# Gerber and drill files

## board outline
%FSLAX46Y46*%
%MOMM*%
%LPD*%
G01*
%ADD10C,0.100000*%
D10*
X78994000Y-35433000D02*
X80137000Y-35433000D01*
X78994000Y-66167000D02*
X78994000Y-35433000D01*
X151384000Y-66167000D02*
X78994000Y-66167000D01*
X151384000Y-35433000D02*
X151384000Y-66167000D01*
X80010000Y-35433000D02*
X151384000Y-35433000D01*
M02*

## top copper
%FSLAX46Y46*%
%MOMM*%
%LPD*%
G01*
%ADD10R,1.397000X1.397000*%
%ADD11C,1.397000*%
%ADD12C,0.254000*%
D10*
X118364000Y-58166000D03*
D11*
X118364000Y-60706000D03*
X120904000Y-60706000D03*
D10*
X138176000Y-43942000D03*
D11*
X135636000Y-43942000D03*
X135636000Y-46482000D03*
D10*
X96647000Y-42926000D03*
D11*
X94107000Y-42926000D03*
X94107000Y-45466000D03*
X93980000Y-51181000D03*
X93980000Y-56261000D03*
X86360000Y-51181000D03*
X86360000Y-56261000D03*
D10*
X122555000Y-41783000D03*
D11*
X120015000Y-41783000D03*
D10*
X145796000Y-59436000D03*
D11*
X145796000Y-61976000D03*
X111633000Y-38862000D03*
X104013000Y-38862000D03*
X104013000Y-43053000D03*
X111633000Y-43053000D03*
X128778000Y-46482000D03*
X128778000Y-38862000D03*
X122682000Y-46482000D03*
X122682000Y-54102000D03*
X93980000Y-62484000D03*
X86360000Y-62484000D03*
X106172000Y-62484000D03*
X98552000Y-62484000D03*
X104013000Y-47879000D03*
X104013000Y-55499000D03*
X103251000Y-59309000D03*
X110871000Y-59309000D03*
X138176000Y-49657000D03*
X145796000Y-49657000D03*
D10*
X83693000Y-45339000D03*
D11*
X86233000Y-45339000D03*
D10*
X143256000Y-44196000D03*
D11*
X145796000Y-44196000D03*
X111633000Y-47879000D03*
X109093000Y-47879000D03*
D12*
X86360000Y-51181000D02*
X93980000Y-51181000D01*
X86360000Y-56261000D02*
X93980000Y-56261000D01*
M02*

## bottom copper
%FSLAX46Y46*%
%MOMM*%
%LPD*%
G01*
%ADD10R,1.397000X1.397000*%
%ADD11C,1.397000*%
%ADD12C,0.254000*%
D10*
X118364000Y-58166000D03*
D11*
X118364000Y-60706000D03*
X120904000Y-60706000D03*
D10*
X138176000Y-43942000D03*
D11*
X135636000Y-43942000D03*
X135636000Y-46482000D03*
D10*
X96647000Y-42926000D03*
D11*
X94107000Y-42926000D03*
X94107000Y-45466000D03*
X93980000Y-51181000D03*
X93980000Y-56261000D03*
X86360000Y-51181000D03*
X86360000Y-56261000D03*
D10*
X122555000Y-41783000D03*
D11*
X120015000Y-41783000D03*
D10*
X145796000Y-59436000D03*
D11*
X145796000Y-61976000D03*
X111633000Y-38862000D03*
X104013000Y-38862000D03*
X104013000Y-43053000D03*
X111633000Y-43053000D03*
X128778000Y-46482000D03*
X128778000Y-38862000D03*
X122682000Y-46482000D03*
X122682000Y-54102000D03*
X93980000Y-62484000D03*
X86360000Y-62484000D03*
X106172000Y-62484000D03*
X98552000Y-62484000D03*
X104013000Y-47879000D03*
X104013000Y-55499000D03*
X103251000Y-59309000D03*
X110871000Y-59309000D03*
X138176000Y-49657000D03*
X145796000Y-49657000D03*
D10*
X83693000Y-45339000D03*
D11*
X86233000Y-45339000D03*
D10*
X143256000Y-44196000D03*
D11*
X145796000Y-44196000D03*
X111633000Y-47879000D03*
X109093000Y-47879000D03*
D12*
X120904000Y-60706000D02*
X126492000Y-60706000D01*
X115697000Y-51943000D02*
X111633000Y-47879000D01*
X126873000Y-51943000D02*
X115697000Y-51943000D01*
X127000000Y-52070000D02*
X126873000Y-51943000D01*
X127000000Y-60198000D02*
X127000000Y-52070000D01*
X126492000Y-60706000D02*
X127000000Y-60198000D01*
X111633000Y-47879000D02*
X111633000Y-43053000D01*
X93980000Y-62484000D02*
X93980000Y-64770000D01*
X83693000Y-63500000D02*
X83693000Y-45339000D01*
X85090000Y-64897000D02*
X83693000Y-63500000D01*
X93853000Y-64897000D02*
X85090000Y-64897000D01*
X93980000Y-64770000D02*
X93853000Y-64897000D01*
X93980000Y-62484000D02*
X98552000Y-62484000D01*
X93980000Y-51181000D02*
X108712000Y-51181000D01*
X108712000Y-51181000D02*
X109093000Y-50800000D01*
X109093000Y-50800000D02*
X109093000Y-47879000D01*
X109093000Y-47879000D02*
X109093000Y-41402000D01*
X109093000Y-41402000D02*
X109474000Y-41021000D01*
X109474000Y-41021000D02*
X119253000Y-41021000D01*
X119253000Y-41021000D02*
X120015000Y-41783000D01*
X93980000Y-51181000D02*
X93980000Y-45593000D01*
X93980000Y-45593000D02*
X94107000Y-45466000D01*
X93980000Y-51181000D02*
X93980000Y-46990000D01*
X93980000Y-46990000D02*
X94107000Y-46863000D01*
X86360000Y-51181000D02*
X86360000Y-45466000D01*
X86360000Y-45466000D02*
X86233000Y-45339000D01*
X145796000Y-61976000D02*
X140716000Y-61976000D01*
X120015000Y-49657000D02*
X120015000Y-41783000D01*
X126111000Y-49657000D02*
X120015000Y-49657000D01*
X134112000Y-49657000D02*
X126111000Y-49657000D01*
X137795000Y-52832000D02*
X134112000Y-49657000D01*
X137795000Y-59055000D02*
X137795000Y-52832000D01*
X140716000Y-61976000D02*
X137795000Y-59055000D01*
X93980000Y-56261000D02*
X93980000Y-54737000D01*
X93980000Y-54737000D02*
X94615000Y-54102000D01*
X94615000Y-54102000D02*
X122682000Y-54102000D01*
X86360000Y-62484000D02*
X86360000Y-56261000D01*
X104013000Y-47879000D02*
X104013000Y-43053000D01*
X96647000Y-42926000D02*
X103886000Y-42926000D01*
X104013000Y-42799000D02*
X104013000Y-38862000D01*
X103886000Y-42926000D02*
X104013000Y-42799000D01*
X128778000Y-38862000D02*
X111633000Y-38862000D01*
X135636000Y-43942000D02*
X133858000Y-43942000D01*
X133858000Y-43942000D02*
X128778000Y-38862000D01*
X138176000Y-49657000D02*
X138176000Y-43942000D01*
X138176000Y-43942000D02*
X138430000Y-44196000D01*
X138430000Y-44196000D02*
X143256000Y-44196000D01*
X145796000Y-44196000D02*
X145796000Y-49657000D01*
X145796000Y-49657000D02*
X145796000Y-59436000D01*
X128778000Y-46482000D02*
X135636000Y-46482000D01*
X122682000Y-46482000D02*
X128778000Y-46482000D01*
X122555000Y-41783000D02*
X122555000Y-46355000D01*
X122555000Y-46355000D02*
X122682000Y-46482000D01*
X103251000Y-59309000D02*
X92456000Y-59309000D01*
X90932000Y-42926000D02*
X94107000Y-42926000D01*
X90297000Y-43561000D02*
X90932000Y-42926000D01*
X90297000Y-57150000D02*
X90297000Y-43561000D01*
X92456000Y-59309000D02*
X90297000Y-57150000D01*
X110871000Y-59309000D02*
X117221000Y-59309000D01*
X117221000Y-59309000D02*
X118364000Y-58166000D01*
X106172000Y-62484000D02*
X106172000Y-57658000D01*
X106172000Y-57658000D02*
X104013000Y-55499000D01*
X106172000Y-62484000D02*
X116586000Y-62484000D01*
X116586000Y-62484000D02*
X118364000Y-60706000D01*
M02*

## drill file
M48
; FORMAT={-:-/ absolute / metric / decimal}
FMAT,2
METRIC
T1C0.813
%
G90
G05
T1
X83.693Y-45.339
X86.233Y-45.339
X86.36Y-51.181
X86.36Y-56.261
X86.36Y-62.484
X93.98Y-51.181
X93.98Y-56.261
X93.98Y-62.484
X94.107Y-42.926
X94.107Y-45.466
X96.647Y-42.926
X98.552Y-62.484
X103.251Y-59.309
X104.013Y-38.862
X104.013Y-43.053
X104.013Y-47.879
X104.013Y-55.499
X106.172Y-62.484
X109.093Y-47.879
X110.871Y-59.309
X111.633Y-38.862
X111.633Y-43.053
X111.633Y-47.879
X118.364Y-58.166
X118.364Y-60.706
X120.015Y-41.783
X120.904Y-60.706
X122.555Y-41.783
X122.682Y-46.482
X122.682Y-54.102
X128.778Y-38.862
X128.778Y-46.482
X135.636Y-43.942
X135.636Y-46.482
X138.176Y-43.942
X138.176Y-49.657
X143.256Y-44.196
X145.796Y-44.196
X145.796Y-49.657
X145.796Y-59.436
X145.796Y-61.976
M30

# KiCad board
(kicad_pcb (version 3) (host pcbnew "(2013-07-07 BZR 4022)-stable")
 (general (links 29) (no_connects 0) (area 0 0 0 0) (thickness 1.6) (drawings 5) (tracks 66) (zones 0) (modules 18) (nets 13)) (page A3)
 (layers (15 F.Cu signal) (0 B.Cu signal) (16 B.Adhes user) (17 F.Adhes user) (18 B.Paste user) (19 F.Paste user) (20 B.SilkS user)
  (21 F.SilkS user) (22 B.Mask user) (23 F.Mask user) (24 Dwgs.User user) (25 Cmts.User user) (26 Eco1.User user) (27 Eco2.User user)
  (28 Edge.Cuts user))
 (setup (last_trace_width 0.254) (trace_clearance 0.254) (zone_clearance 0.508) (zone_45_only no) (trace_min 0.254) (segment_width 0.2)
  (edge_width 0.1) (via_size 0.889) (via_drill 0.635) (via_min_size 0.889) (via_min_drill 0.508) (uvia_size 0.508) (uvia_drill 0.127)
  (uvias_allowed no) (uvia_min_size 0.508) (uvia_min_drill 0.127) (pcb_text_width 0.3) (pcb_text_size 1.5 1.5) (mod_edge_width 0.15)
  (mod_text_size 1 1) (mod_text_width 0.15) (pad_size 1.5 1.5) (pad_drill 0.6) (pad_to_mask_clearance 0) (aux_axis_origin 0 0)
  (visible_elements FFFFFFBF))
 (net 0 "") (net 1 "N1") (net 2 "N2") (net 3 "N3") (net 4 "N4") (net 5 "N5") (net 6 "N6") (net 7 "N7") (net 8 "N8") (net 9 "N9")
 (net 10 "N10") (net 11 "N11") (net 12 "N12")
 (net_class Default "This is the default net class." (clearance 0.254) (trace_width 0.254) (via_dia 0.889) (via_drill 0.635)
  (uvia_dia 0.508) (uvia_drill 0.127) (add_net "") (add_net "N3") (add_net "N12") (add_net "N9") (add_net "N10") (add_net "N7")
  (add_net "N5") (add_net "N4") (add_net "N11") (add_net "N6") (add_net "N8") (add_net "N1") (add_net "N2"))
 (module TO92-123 (layer F.Cu) (at 119.634 59.436 90)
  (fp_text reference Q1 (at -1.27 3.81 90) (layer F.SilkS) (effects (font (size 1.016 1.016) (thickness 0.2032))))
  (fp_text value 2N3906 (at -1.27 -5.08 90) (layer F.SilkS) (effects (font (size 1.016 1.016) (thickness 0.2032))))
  (pad 3 thru_hole rect (at 1.27 -1.27 90) (size 1.397 1.397) (drill 0.8128) (layers *.Cu *.Mask F.SilkS) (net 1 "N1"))
  (pad 2 thru_hole circle (at -1.27 -1.27 90) (size 1.397 1.397) (drill 0.8128) (layers *.Cu *.Mask F.SilkS) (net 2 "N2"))
  (pad 1 thru_hole circle (at -1.27 1.27 90) (size 1.397 1.397) (drill 0.8128) (layers *.Cu *.Mask F.SilkS) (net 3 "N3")))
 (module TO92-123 (layer F.Cu) (at 136.906 45.212)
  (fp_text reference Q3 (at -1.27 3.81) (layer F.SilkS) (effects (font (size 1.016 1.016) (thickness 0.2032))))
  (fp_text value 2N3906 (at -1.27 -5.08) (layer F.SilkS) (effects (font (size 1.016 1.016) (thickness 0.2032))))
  (pad 3 thru_hole rect (at 1.27 -1.27) (size 1.397 1.397) (drill 0.8128) (layers *.Cu *.Mask F.SilkS) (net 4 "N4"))
  (pad 2 thru_hole circle (at -1.27 -1.27) (size 1.397 1.397) (drill 0.8128) (layers *.Cu *.Mask F.SilkS) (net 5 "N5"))
  (pad 1 thru_hole circle (at -1.27 1.27) (size 1.397 1.397) (drill 0.8128) (layers *.Cu *.Mask F.SilkS) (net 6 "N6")))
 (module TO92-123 (layer F.Cu) (at 95.377 44.196)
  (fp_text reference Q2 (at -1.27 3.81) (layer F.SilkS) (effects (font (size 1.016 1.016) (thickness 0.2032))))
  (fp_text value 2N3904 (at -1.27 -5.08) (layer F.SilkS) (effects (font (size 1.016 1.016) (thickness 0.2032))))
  (pad 3 thru_hole rect (at 1.27 -1.27) (size 1.397 1.397) (drill 0.8128) (layers *.Cu *.Mask F.SilkS) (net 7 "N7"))
  (pad 2 thru_hole circle (at -1.27 -1.27) (size 1.397 1.397) (drill 0.8128) (layers *.Cu *.Mask F.SilkS) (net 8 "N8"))
  (pad 1 thru_hole circle (at -1.27 1.27) (size 1.397 1.397) (drill 0.8128) (layers *.Cu *.Mask F.SilkS) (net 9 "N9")))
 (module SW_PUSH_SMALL (layer F.Cu) (at 90.17 53.721)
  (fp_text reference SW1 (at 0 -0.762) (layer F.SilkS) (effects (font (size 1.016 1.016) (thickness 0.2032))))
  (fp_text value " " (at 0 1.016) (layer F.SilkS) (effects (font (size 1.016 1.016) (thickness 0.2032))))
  (pad 1 thru_hole circle (at 3.81 -2.54) (size 1.397 1.397) (drill 0.8128) (layers *.Cu *.Mask F.SilkS) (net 9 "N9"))
  (pad 2 thru_hole circle (at 3.81 2.54) (size 1.397 1.397) (drill 0.8128) (layers *.Cu *.Mask F.SilkS) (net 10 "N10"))
  (pad 1 thru_hole circle (at -3.81 -2.54) (size 1.397 1.397) (drill 0.8128) (layers *.Cu *.Mask F.SilkS) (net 9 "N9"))
  (pad 2 thru_hole circle (at -3.81 2.54) (size 1.397 1.397) (drill 0.8128) (layers *.Cu *.Mask F.SilkS) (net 10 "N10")))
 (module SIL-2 (layer F.Cu) (at 121.285 41.783 180)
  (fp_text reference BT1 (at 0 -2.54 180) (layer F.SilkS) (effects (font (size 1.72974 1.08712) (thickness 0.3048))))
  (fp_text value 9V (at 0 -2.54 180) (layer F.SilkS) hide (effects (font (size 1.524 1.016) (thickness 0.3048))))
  (pad 1 thru_hole rect (at -1.27 0 180) (size 1.397 1.397) (drill 0.8128) (layers *.Cu *.Mask F.SilkS) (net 6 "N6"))
  (pad 2 thru_hole circle (at 1.27 0 180) (size 1.397 1.397) (drill 0.8128) (layers *.Cu *.Mask F.SilkS) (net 9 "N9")))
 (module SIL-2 (layer F.Cu) (at 145.796 60.706 270)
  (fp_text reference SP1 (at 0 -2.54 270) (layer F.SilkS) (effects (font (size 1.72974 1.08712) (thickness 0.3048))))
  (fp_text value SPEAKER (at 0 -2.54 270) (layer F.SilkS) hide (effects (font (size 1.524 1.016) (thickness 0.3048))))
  (pad 1 thru_hole rect (at -1.27 0 270) (size 1.397 1.397) (drill 0.8128) (layers *.Cu *.Mask F.SilkS) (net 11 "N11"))
  (pad 2 thru_hole circle (at 1.27 0 270) (size 1.397 1.397) (drill 0.8128) (layers *.Cu *.Mask F.SilkS) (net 9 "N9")))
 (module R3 (layer F.Cu) (at 107.823 38.862 180) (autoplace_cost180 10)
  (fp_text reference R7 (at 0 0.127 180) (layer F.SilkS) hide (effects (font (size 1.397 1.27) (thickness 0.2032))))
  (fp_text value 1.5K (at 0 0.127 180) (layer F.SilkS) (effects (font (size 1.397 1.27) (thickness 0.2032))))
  (pad 1 thru_hole circle (at -3.81 0 180) (size 1.397 1.397) (drill 0.8128) (layers *.Cu *.Mask F.SilkS) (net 5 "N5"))
  (pad 2 thru_hole circle (at 3.81 0 180) (size 1.397 1.397) (drill 0.8128) (layers *.Cu *.Mask F.SilkS) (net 7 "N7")))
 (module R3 (layer F.Cu) (at 107.823 43.053) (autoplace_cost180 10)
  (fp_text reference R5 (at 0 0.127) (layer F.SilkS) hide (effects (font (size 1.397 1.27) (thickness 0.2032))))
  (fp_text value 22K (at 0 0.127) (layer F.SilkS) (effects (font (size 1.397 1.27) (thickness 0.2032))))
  (pad 1 thru_hole circle (at -3.81 0) (size 1.397 1.397) (drill 0.8128) (layers *.Cu *.Mask F.SilkS) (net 7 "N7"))
  (pad 2 thru_hole circle (at 3.81 0) (size 1.397 1.397) (drill 0.8128) (layers *.Cu *.Mask F.SilkS) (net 3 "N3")))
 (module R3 (layer F.Cu) (at 128.778 42.672 90) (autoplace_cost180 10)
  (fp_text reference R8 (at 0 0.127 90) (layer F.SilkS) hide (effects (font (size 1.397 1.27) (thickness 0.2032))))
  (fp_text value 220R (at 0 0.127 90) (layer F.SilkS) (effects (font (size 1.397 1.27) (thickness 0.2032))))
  (pad 1 thru_hole circle (at -3.81 0 90) (size 1.397 1.397) (drill 0.8128) (layers *.Cu *.Mask F.SilkS) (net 6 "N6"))
  (pad 2 thru_hole circle (at 3.81 0 90) (size 1.397 1.397) (drill 0.8128) (layers *.Cu *.Mask F.SilkS) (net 5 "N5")))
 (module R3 (layer F.Cu) (at 122.682 50.292 270) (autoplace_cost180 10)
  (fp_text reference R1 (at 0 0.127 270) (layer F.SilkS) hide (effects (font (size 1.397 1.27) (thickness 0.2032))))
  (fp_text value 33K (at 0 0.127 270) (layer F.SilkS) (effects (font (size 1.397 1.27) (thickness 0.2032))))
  (pad 1 thru_hole circle (at -3.81 0 270) (size 1.397 1.397) (drill 0.8128) (layers *.Cu *.Mask F.SilkS) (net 6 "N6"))
  (pad 2 thru_hole circle (at 3.81 0 270) (size 1.397 1.397) (drill 0.8128) (layers *.Cu *.Mask F.SilkS) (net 10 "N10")))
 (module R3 (layer F.Cu) (at 90.17 62.484 180) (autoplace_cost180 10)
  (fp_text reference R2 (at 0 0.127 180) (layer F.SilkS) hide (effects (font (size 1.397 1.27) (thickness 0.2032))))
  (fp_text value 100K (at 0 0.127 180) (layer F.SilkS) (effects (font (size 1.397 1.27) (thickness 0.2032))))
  (pad 1 thru_hole circle (at -3.81 0 180) (size 1.397 1.397) (drill 0.8128) (layers *.Cu *.Mask F.SilkS) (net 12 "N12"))
  (pad 2 thru_hole circle (at 3.81 0 180) (size 1.397 1.397) (drill 0.8128) (layers *.Cu *.Mask F.SilkS) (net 10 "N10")))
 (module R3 (layer F.Cu) (at 102.362 62.484 180) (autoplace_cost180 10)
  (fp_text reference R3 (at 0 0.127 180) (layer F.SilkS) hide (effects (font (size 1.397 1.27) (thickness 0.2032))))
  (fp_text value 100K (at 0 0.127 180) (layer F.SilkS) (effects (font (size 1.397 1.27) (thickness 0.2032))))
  (pad 1 thru_hole circle (at -3.81 0 180) (size 1.397 1.397) (drill 0.8128) (layers *.Cu *.Mask F.SilkS) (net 2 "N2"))
  (pad 2 thru_hole circle (at 3.81 0 180) (size 1.397 1.397) (drill 0.8128) (layers *.Cu *.Mask F.SilkS) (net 12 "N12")))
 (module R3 (layer F.Cu) (at 104.013 51.689 270) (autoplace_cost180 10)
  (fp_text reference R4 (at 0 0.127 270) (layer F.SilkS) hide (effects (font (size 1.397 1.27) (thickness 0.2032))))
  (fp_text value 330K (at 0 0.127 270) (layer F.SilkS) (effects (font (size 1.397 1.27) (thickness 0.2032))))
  (pad 1 thru_hole circle (at -3.81 0 270) (size 1.397 1.397) (drill 0.8128) (layers *.Cu *.Mask F.SilkS) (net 7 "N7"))
  (pad 2 thru_hole circle (at 3.81 0 270) (size 1.397 1.397) (drill 0.8128) (layers *.Cu *.Mask F.SilkS) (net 2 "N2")))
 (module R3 (layer F.Cu) (at 107.061 59.309) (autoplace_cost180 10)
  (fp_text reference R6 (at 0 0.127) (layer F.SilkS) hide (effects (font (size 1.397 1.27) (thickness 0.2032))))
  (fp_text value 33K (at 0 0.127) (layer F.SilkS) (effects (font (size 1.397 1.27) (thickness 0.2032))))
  (pad 1 thru_hole circle (at -3.81 0) (size 1.397 1.397) (drill 0.8128) (layers *.Cu *.Mask F.SilkS) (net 8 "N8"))
  (pad 2 thru_hole circle (at 3.81 0) (size 1.397 1.397) (drill 0.8128) (layers *.Cu *.Mask F.SilkS) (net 1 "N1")))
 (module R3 (layer F.Cu) (at 141.986 49.657) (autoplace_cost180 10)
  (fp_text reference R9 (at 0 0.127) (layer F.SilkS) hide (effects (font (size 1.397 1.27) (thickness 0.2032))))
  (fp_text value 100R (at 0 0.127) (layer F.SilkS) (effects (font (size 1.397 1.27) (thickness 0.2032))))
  (pad 1 thru_hole circle (at -3.81 0) (size 1.397 1.397) (drill 0.8128) (layers *.Cu *.Mask F.SilkS) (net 4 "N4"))
  (pad 2 thru_hole circle (at 3.81 0) (size 1.397 1.397) (drill 0.8128) (layers *.Cu *.Mask F.SilkS) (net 11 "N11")))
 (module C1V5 (layer F.Cu) (at 84.963 45.339)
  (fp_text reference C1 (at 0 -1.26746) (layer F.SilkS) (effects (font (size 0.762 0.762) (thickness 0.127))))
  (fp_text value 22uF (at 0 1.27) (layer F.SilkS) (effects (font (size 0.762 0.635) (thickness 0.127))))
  (pad 1 thru_hole rect (at -1.27 0) (size 1.397 1.397) (drill 0.8128) (layers *.Cu *.Mask F.SilkS) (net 12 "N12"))
  (pad 2 thru_hole circle (at 1.27 0) (size 1.397 1.397) (drill 0.8128) (layers *.Cu *.Mask F.SilkS) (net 9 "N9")))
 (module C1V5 (layer F.Cu) (at 144.526 44.196)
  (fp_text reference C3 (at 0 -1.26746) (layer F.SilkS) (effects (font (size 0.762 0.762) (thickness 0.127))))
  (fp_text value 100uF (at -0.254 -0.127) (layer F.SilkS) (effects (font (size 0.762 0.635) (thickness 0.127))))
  (pad 1 thru_hole rect (at -1.27 0) (size 1.397 1.397) (drill 0.8128) (layers *.Cu *.Mask F.SilkS) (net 4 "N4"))
  (pad 2 thru_hole circle (at 1.27 0) (size 1.397 1.397) (drill 0.8128) (layers *.Cu *.Mask F.SilkS) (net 11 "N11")))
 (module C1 (layer F.Cu) (at 110.363 47.879 180)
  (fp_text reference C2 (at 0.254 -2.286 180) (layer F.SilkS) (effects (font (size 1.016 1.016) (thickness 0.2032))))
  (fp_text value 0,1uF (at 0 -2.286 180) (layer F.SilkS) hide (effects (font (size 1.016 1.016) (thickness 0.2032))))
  (pad 1 thru_hole circle (at -1.27 0 180) (size 1.397 1.397) (drill 0.8128) (layers *.Cu *.Mask F.SilkS) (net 3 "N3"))
  (pad 2 thru_hole circle (at 1.27 0 180) (size 1.397 1.397) (drill 0.8128) (layers *.Cu *.Mask F.SilkS) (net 9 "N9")))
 (gr_line (start 78.994 35.433) (end 80.137 35.433) (angle 90) (layer Edge.Cuts) (width 0.1))
 (gr_line (start 78.994 66.167) (end 78.994 35.433) (angle 90) (layer Edge.Cuts) (width 0.1))
 (gr_line (start 151.384 66.167) (end 78.994 66.167) (angle 90) (layer Edge.Cuts) (width 0.1))
 (gr_line (start 151.384 35.433) (end 151.384 66.167) (angle 90) (layer Edge.Cuts) (width 0.1))
 (gr_line (start 80.01 35.433) (end 151.384 35.433) (angle 90) (layer Edge.Cuts) (width 0.1))
 (segment (start 120.904 60.706) (end 126.492 60.706) (width 0.254) (layer B.Cu) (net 3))
 (segment (start 115.697 51.943) (end 111.633 47.879) (width 0.254) (layer B.Cu) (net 3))
 (segment (start 126.873 51.943) (end 115.697 51.943) (width 0.254) (layer B.Cu) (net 3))
 (segment (start 127 52.07) (end 126.873 51.943) (width 0.254) (layer B.Cu) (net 3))
 (segment (start 127 60.198) (end 127 52.07) (width 0.254) (layer B.Cu) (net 3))
 (segment (start 126.492 60.706) (end 127 60.198) (width 0.254) (layer B.Cu) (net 3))
 (segment (start 111.633 47.879) (end 111.633 43.053) (width 0.254) (layer B.Cu) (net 3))
 (segment (start 93.98 62.484) (end 93.98 64.77) (width 0.254) (layer B.Cu) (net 12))
 (segment (start 83.693 63.5) (end 83.693 45.339) (width 0.254) (layer B.Cu) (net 12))
 (segment (start 85.09 64.897) (end 83.693 63.5) (width 0.254) (layer B.Cu) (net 12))
 (segment (start 93.853 64.897) (end 85.09 64.897) (width 0.254) (layer B.Cu) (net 12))
 (segment (start 93.98 64.77) (end 93.853 64.897) (width 0.254) (layer B.Cu) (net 12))
 (segment (start 93.98 62.484) (end 98.552 62.484) (width 0.254) (layer B.Cu) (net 12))
 (segment (start 86.36 51.181) (end 93.98 51.181) (width 0.254) (layer F.Cu) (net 9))
 (segment (start 93.98 51.181) (end 108.712 51.181) (width 0.254) (layer B.Cu) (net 9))
 (segment (start 108.712 51.181) (end 109.093 50.8) (width 0.254) (layer B.Cu) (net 9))
 (segment (start 109.093 50.8) (end 109.093 47.879) (width 0.254) (layer B.Cu) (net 9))
 (segment (start 109.093 47.879) (end 109.093 41.402) (width 0.254) (layer B.Cu) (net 9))
 (segment (start 109.093 41.402) (end 109.474 41.021) (width 0.254) (layer B.Cu) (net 9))
 (segment (start 109.474 41.021) (end 119.253 41.021) (width 0.254) (layer B.Cu) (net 9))
 (segment (start 119.253 41.021) (end 120.015 41.783) (width 0.254) (layer B.Cu) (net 9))
 (segment (start 93.98 51.181) (end 93.98 45.593) (width 0.254) (layer B.Cu) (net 9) (status 10))
 (segment (start 93.98 45.593) (end 94.107 45.466) (width 0.254) (layer B.Cu) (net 9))
 (segment (start 93.98 51.181) (end 93.98 46.99) (width 0.254) (layer B.Cu) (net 9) (status 10))
 (segment (start 93.98 46.99) (end 94.107 46.863) (width 0.254) (layer B.Cu) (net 9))
 (segment (start 86.36 51.181) (end 86.36 45.466) (width 0.254) (layer B.Cu) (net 9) (status 10))
 (segment (start 86.36 45.466) (end 86.233 45.339) (width 0.254) (layer B.Cu) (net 9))
 (segment (start 145.796 61.976) (end 140.716 61.976) (width 0.254) (layer B.Cu) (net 9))
 (segment (start 120.015 49.657) (end 120.015 41.783) (width 0.254) (layer B.Cu) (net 9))
 (segment (start 126.111 49.657) (end 120.015 49.657) (width 0.254) (layer B.Cu) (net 9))
 (segment (start 134.112 49.657) (end 126.111 49.657) (width 0.254) (layer B.Cu) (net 9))
 (segment (start 137.795 52.832) (end 134.112 49.657) (width 0.254) (layer B.Cu) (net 9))
 (segment (start 137.795 59.055) (end 137.795 52.832) (width 0.254) (layer B.Cu) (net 9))
 (segment (start 140.716 61.976) (end 137.795 59.055) (width 0.254) (layer B.Cu) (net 9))
 (segment (start 86.36 56.261) (end 93.98 56.261) (width 0.254) (layer F.Cu) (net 10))
 (segment (start 93.98 56.261) (end 93.98 54.737) (width 0.254) (layer B.Cu) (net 10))
 (segment (start 93.98 54.737) (end 94.615 54.102) (width 0.254) (layer B.Cu) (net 10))
 (segment (start 94.615 54.102) (end 122.682 54.102) (width 0.254) (layer B.Cu) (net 10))
 (segment (start 86.36 62.484) (end 86.36 56.261) (width 0.254) (layer B.Cu) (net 10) (status 20))
 (segment (start 104.013 47.879) (end 104.013 43.053) (width 0.254) (layer B.Cu) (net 7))
 (segment (start 96.647 42.926) (end 103.886 42.926) (width 0.254) (layer B.Cu) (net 7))
 (segment (start 104.013 42.799) (end 104.013 38.862) (width 0.254) (layer B.Cu) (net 7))
 (segment (start 103.886 42.926) (end 104.013 42.799) (width 0.254) (layer B.Cu) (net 7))
 (segment (start 128.778 38.862) (end 111.633 38.862) (width 0.254) (layer B.Cu) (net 5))
 (segment (start 135.636 43.942) (end 133.858 43.942) (width 0.254) (layer B.Cu) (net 5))
 (segment (start 133.858 43.942) (end 128.778 38.862) (width 0.254) (layer B.Cu) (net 5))
 (segment (start 138.176 49.657) (end 138.176 43.942) (width 0.254) (layer B.Cu) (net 4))
 (segment (start 138.176 43.942) (end 138.43 44.196) (width 0.254) (layer B.Cu) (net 4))
 (segment (start 138.43 44.196) (end 143.256 44.196) (width 0.254) (layer B.Cu) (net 4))
 (segment (start 145.796 44.196) (end 145.796 49.657) (width 0.254) (layer B.Cu) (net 11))
 (segment (start 145.796 49.657) (end 145.796 59.436) (width 0.254) (layer B.Cu) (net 11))
 (segment (start 128.778 46.482) (end 135.636 46.482) (width 0.254) (layer B.Cu) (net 6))
 (segment (start 122.682 46.482) (end 128.778 46.482) (width 0.254) (layer B.Cu) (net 6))
 (segment (start 122.555 41.783) (end 122.555 46.355) (width 0.254) (layer B.Cu) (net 6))
 (segment (start 122.555 46.355) (end 122.682 46.482) (width 0.254) (layer B.Cu) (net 6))
 (segment (start 103.251 59.309) (end 92.456 59.309) (width 0.254) (layer B.Cu) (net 8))
 (segment (start 90.932 42.926) (end 94.107 42.926) (width 0.254) (layer B.Cu) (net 8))
 (segment (start 90.297 43.561) (end 90.932 42.926) (width 0.254) (layer B.Cu) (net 8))
 (segment (start 90.297 57.15) (end 90.297 43.561) (width 0.254) (layer B.Cu) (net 8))
 (segment (start 92.456 59.309) (end 90.297 57.15) (width 0.254) (layer B.Cu) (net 8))
 (segment (start 110.871 59.309) (end 117.221 59.309) (width 0.254) (layer B.Cu) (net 1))
 (segment (start 117.221 59.309) (end 118.364 58.166) (width 0.254) (layer B.Cu) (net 1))
 (segment (start 106.172 62.484) (end 106.172 57.658) (width 0.254) (layer B.Cu) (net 2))
 (segment (start 106.172 57.658) (end 104.013 55.499) (width 0.254) (layer B.Cu) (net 2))
 (segment (start 106.172 62.484) (end 116.586 62.484) (width 0.254) (layer B.Cu) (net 2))
 (segment (start 116.586 62.484) (end 118.364 60.706) (width 0.254) (layer B.Cu) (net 2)))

